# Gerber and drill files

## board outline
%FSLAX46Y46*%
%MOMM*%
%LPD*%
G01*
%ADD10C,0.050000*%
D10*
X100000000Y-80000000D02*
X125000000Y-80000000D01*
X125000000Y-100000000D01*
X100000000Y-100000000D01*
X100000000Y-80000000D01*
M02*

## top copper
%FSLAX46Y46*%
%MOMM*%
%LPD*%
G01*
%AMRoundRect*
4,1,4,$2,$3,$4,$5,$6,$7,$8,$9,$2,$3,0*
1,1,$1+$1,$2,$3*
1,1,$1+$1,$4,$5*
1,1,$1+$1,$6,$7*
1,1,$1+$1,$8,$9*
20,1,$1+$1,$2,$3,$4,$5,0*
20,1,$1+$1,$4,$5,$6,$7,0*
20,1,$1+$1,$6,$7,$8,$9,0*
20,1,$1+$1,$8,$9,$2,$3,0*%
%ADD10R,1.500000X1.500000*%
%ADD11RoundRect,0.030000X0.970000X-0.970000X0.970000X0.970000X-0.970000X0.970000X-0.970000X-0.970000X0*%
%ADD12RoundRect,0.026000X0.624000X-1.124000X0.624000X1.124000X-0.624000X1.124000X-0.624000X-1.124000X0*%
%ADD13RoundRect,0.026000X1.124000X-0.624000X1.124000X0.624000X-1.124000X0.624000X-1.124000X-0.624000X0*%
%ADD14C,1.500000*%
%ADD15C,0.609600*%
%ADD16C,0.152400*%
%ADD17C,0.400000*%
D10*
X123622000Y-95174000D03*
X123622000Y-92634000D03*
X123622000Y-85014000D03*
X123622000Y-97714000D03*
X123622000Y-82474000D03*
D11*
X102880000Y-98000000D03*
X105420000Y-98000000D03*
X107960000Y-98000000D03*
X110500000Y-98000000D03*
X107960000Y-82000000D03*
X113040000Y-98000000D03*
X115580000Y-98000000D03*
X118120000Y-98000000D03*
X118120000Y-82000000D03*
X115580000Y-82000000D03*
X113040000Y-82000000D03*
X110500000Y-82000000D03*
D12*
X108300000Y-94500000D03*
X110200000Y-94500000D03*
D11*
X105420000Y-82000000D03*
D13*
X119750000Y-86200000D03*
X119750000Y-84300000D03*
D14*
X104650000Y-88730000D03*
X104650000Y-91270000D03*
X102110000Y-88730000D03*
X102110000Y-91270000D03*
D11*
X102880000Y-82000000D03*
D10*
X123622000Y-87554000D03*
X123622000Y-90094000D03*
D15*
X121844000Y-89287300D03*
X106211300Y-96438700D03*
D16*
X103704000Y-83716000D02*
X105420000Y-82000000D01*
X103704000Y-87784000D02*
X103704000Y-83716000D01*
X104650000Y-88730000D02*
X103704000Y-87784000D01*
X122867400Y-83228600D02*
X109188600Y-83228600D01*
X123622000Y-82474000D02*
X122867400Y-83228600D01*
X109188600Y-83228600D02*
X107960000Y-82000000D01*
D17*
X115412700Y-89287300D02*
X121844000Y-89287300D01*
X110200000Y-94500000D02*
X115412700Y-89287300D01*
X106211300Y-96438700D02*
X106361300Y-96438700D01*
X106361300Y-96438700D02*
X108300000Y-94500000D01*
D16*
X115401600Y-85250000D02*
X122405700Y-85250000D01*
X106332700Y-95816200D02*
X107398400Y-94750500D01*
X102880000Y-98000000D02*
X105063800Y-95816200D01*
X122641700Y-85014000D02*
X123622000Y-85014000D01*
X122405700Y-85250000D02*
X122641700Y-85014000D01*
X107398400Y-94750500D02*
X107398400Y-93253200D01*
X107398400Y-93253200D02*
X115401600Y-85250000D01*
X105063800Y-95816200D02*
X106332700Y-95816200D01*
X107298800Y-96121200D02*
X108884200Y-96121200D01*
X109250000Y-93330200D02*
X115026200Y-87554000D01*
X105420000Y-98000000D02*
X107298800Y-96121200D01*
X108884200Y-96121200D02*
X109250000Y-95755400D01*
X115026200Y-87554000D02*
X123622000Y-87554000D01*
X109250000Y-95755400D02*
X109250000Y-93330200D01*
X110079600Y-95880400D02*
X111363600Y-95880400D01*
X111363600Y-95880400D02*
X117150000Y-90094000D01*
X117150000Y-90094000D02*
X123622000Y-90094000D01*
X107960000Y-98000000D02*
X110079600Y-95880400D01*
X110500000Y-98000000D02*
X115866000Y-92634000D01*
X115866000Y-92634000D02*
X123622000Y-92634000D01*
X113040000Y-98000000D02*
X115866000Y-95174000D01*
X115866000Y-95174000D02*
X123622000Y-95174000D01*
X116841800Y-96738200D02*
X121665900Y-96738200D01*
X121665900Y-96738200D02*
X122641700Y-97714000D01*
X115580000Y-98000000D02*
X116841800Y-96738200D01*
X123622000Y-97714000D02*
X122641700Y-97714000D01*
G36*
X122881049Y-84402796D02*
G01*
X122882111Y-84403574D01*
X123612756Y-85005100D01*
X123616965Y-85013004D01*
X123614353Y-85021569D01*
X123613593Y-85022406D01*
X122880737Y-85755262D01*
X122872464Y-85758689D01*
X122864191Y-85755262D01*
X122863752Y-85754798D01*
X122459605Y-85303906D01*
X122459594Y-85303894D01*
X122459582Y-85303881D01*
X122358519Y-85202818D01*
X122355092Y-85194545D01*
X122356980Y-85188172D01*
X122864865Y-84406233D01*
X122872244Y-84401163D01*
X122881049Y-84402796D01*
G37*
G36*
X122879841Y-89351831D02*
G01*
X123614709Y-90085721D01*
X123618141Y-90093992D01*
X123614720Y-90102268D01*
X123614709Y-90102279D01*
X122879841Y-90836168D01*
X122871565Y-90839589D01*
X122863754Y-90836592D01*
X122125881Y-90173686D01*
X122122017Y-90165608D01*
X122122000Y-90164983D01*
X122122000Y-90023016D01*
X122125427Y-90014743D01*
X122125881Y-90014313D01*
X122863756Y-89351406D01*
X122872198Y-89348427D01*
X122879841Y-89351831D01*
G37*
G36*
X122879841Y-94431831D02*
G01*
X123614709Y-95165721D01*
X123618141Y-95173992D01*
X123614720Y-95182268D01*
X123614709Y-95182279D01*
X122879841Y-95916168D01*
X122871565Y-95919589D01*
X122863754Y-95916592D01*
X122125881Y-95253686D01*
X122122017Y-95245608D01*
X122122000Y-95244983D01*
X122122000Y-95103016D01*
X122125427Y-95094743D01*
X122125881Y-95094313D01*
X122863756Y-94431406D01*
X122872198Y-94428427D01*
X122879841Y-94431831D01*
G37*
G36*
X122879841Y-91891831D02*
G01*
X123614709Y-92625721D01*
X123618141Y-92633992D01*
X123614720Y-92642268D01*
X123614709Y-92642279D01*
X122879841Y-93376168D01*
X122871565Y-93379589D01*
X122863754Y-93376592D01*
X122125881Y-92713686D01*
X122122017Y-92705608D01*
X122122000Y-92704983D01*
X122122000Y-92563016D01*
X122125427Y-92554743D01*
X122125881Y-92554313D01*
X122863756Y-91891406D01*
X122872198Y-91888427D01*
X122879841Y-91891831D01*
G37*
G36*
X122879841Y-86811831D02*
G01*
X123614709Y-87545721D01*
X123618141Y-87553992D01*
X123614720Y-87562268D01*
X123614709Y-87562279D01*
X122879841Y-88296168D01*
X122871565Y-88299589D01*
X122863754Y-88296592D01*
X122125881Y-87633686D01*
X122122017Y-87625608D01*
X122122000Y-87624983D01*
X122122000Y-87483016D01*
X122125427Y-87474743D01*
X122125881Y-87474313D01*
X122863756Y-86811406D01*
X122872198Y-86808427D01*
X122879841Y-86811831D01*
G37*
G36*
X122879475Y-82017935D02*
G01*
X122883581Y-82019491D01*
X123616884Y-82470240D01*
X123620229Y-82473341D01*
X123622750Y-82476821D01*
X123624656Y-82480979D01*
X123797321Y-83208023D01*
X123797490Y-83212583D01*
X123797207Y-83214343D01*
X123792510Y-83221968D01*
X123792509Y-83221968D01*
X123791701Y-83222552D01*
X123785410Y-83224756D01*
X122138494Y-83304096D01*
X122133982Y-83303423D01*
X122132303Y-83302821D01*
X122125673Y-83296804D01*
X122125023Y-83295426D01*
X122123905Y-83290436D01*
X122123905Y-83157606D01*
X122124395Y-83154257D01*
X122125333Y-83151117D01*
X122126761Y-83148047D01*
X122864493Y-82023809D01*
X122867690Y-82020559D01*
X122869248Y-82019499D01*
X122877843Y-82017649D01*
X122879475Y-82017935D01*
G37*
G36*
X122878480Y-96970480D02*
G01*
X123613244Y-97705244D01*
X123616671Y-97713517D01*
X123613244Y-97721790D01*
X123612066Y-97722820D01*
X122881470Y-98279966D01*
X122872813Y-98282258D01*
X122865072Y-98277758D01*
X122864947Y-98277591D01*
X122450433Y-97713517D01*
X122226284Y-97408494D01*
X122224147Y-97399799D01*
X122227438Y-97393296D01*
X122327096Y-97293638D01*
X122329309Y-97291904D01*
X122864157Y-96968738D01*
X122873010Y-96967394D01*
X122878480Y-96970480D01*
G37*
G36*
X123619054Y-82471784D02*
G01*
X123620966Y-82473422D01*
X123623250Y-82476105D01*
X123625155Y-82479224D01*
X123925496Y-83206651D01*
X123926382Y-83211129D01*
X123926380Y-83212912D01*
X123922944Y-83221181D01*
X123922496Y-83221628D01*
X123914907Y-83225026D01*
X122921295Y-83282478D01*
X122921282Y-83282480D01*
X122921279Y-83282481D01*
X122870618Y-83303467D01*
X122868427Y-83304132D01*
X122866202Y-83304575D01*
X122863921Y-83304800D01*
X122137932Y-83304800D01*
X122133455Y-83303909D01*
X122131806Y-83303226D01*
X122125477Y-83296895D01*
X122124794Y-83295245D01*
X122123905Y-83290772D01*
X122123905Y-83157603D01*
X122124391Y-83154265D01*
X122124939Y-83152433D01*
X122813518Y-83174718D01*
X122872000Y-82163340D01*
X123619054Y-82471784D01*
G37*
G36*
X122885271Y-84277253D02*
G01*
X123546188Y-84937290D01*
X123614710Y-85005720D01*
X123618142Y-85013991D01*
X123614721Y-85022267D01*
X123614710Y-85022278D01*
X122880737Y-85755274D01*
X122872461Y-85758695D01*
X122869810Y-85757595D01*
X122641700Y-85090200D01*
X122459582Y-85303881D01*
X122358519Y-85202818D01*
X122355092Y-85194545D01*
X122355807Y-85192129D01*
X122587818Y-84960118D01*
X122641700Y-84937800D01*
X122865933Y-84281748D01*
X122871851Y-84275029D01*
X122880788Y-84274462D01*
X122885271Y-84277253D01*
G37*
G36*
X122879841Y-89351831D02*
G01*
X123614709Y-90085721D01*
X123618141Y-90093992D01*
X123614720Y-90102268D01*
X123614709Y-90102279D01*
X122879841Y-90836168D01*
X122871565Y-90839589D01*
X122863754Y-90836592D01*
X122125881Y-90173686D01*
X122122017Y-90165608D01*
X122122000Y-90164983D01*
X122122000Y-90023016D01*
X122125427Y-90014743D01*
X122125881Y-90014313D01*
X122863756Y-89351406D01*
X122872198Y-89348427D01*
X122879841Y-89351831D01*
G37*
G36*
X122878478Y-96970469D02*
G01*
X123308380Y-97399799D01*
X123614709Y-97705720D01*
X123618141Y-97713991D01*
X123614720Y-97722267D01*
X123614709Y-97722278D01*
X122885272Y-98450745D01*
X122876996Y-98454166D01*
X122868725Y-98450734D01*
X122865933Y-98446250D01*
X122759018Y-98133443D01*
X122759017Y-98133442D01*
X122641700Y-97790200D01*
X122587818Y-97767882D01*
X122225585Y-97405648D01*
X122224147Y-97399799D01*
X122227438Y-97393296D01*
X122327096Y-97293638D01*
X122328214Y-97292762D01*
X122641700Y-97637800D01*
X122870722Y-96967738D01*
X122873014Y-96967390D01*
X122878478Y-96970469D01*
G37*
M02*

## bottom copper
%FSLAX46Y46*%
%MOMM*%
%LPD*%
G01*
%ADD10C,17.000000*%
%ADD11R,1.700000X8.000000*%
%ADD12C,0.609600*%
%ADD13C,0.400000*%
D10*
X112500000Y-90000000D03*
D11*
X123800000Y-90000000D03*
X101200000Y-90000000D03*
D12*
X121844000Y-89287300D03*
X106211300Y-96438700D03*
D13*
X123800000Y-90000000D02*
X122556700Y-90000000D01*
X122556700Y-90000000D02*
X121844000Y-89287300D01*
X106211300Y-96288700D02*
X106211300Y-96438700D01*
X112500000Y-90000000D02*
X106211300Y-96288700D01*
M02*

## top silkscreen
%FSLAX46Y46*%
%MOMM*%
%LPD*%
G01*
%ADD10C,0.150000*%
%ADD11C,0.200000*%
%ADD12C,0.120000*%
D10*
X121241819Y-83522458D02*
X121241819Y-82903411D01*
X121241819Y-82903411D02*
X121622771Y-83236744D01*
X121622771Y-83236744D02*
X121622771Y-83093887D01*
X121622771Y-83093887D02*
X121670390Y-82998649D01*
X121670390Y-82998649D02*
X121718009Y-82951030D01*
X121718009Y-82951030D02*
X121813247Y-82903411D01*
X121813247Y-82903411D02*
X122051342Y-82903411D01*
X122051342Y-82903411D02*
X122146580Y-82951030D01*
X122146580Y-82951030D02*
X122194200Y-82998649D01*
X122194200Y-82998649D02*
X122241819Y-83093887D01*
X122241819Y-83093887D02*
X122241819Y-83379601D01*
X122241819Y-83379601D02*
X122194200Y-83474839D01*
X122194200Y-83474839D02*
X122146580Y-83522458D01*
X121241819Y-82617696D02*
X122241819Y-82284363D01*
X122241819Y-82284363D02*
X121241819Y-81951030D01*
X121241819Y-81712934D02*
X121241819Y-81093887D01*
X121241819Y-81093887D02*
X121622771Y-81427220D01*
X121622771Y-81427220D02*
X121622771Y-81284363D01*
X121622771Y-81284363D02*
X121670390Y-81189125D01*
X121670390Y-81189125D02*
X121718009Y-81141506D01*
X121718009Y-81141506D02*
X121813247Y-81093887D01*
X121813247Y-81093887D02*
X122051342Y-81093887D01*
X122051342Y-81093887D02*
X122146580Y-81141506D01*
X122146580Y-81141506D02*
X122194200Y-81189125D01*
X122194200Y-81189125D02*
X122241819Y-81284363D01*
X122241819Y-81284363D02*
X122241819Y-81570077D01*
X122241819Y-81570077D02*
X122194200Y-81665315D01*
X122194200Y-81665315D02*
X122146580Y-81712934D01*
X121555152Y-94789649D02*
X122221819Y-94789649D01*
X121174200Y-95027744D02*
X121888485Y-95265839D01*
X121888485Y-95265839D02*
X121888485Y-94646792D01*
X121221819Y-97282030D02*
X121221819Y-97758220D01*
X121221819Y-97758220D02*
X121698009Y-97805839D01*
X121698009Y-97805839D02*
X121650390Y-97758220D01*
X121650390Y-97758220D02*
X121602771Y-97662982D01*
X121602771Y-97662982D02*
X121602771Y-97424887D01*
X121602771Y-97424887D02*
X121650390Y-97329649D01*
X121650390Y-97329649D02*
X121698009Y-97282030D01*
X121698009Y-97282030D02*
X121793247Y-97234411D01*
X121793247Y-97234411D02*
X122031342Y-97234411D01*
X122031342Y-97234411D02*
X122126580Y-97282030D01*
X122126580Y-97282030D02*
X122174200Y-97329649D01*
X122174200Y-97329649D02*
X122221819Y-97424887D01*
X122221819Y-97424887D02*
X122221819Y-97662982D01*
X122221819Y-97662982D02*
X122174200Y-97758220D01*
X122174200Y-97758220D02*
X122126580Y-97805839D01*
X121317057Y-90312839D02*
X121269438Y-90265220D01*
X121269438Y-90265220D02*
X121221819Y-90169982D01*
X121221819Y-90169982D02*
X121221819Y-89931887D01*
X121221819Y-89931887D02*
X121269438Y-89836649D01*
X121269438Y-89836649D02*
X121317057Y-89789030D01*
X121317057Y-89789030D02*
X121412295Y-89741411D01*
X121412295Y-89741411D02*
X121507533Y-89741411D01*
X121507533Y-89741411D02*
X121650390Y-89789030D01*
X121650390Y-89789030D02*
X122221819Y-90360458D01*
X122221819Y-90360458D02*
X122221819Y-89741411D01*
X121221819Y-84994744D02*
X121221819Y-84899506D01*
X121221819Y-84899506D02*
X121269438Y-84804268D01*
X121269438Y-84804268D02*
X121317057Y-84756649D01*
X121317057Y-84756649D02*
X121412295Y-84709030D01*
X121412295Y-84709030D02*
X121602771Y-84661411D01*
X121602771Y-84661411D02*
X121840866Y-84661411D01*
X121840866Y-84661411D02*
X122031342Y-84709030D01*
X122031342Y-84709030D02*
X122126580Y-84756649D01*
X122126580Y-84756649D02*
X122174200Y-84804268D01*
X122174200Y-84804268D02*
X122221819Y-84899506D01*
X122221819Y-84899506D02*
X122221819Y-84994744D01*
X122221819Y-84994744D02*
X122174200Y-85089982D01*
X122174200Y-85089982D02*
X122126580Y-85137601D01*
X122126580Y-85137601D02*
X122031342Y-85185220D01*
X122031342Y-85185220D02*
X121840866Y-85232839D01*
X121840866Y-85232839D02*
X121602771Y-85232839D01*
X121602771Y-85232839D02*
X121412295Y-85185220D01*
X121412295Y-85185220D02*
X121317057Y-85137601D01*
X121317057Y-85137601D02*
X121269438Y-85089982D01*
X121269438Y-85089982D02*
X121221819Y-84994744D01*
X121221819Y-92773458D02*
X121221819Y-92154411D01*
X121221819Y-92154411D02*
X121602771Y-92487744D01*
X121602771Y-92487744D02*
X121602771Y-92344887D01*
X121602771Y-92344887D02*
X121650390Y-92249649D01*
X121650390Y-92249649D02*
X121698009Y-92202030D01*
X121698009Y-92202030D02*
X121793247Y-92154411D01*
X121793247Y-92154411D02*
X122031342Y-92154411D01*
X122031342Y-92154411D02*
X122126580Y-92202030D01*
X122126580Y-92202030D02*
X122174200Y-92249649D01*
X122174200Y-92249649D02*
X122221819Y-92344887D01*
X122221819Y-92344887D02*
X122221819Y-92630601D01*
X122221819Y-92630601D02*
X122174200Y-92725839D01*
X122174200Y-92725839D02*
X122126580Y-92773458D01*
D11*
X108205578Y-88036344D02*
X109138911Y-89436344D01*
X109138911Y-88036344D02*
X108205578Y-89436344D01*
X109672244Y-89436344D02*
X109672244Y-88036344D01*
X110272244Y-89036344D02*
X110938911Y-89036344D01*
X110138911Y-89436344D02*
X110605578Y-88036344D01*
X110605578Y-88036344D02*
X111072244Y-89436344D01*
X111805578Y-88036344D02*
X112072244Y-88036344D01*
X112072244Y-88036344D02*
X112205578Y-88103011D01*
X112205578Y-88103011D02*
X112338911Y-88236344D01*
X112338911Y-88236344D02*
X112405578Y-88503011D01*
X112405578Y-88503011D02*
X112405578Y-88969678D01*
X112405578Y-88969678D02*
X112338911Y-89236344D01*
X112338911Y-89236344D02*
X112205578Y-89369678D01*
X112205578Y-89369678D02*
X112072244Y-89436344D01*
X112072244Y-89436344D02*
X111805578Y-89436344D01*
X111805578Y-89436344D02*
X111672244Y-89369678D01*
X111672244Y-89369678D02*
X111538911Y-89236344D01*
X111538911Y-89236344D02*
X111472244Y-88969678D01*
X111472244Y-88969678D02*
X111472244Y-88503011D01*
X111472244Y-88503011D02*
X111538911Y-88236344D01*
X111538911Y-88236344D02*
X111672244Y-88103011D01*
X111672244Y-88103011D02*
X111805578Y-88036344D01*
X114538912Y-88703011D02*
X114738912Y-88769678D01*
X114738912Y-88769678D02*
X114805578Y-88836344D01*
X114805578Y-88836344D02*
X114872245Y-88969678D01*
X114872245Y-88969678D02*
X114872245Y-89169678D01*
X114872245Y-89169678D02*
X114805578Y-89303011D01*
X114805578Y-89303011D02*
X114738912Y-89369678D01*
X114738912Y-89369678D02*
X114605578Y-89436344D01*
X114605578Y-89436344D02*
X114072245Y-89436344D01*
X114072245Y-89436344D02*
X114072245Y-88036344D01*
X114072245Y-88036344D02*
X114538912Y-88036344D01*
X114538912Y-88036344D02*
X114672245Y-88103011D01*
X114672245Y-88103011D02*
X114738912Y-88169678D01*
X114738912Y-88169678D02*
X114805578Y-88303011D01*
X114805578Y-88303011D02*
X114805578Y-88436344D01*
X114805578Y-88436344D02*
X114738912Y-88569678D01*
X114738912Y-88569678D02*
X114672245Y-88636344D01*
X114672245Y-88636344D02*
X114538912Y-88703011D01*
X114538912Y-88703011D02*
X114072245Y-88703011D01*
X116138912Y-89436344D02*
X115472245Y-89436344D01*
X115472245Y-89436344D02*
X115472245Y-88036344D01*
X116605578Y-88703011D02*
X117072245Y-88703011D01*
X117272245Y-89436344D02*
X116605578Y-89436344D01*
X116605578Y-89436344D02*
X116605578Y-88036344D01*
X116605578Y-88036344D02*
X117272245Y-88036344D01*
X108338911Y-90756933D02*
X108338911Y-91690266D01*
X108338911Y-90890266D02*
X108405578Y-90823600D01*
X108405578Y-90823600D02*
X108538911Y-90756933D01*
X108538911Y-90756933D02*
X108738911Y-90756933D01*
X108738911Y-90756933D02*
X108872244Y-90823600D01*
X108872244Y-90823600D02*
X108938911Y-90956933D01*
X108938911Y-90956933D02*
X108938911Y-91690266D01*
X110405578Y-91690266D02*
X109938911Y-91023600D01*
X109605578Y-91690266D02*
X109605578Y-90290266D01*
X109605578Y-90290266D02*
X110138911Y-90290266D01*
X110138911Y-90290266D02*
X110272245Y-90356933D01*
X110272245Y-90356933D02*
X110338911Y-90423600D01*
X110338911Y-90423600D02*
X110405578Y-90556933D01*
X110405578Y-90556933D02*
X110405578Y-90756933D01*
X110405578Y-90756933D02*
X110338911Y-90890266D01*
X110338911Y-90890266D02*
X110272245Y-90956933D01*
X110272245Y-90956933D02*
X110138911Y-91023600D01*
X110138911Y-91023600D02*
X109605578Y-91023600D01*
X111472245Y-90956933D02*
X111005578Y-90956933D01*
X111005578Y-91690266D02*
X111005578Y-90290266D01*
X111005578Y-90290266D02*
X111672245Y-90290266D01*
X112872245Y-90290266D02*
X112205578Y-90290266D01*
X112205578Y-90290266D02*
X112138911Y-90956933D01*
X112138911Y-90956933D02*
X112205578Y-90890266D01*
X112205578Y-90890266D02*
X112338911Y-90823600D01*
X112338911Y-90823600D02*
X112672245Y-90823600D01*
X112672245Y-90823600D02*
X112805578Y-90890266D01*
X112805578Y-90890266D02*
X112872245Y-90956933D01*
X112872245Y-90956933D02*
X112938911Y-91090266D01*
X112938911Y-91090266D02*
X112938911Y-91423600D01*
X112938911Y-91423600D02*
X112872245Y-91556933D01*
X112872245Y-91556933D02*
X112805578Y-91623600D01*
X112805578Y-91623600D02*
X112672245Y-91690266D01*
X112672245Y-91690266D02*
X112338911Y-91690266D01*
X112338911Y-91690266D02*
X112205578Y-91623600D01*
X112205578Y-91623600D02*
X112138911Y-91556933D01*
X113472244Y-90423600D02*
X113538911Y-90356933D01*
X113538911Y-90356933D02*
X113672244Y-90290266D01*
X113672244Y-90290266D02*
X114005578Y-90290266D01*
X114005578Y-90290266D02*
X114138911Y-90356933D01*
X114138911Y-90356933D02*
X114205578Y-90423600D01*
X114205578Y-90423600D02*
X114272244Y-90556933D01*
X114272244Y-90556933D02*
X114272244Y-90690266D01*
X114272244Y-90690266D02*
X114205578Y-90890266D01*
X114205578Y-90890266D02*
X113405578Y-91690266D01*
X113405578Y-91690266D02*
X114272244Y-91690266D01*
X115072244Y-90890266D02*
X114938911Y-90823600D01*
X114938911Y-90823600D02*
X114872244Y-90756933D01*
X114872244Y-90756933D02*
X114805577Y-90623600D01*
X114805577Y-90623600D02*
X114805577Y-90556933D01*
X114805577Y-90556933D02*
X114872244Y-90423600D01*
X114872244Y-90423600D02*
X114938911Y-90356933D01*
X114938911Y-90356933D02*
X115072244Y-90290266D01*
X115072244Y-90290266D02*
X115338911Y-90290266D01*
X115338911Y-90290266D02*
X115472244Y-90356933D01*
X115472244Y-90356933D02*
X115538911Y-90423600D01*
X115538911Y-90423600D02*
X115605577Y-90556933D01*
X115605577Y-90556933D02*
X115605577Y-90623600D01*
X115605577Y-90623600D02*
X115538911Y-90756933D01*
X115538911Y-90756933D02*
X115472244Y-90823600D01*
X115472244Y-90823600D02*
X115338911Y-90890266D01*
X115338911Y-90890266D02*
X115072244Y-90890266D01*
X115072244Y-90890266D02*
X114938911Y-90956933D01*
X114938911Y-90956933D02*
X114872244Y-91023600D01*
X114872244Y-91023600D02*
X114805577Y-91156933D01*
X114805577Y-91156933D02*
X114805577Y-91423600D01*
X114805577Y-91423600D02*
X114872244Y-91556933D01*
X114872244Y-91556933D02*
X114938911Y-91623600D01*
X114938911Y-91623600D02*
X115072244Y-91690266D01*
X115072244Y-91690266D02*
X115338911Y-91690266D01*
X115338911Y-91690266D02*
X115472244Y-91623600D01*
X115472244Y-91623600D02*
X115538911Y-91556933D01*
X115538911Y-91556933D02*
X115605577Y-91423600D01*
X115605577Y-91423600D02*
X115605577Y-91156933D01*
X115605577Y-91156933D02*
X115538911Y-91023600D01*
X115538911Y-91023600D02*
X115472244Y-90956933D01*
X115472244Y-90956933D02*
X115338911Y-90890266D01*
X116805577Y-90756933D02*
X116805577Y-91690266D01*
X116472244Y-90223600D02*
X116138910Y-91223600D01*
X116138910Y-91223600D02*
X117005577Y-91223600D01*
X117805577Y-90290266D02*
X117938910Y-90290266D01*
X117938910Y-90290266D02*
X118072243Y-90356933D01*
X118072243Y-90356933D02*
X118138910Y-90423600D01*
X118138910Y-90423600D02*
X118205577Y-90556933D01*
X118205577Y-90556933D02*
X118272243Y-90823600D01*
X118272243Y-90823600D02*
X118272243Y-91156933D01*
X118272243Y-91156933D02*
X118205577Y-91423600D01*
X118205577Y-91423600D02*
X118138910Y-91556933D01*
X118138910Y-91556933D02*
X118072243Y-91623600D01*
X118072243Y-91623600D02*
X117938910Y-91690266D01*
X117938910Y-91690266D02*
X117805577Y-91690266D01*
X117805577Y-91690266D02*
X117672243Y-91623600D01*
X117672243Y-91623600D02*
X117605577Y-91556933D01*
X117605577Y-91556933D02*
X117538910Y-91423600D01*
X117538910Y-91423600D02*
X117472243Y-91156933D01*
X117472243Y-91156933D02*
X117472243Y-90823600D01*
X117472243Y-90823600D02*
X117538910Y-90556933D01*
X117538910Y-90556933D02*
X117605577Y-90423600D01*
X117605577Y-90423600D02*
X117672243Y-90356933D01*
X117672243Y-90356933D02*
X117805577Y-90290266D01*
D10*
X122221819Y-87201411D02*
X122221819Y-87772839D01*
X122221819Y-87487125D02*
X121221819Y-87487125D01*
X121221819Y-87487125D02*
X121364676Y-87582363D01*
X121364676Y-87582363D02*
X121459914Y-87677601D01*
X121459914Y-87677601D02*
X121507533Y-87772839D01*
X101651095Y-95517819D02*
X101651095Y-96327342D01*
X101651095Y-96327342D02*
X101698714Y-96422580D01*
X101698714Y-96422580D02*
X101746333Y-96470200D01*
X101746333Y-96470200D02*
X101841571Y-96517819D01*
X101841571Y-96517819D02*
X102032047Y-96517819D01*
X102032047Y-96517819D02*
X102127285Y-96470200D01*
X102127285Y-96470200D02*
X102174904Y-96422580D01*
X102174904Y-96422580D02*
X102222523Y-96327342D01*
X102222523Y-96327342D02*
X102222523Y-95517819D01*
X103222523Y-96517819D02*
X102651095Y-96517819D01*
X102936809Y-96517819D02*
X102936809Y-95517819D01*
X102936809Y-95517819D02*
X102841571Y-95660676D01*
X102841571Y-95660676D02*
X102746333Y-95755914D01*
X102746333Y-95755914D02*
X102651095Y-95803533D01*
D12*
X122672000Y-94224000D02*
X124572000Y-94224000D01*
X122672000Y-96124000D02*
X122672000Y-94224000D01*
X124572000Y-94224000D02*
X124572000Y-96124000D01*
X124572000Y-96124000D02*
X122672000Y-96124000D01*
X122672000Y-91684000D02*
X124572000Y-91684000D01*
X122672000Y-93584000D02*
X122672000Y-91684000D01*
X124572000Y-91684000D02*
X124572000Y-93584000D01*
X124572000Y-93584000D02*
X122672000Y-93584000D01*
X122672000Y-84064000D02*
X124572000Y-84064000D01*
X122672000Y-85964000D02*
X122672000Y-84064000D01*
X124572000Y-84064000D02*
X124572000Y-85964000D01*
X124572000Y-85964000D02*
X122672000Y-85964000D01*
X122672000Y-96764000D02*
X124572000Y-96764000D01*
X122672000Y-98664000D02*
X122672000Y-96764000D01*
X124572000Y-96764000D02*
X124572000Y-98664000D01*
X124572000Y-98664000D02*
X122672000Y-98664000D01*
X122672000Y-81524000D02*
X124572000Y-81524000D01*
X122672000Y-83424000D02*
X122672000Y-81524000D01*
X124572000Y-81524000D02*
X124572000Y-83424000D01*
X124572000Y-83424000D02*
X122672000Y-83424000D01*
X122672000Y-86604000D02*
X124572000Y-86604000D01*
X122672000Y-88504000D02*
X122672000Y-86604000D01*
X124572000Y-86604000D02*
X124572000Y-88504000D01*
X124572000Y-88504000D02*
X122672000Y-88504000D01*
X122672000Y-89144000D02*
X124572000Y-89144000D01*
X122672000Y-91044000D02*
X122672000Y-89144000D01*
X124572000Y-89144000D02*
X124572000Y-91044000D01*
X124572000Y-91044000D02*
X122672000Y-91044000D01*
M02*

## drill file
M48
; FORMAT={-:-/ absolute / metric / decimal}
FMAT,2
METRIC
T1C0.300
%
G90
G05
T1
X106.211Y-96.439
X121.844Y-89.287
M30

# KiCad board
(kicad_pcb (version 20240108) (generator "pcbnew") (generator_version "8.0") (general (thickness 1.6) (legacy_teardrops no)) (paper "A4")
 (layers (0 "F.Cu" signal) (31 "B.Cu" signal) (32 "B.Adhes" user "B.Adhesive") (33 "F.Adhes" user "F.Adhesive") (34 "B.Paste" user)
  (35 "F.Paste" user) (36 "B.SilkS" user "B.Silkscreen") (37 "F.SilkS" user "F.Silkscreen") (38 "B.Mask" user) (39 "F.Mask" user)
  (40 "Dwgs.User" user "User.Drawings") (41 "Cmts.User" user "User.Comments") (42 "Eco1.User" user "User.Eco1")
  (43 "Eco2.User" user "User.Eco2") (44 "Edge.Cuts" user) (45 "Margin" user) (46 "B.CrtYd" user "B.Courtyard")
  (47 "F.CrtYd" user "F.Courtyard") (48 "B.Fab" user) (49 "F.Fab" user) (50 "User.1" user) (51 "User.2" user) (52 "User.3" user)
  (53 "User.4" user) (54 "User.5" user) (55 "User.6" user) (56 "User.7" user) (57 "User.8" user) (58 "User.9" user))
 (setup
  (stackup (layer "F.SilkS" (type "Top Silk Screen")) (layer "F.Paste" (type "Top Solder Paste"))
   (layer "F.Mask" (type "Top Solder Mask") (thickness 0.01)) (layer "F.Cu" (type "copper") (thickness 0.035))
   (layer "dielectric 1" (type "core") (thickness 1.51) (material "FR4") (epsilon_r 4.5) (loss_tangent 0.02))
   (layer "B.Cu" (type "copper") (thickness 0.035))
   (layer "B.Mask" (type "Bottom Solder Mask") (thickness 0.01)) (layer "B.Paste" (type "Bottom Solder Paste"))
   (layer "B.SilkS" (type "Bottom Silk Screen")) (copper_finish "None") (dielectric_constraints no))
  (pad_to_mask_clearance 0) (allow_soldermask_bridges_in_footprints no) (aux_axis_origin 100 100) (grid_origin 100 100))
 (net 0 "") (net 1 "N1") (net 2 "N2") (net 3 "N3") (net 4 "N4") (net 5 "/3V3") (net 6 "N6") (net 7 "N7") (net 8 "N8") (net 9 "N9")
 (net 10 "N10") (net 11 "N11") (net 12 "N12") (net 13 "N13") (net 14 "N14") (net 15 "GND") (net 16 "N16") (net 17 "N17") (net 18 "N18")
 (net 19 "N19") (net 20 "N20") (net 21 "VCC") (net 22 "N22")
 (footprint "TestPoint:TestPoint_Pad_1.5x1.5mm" (layer "F.Cu") (at 123.622 95.174)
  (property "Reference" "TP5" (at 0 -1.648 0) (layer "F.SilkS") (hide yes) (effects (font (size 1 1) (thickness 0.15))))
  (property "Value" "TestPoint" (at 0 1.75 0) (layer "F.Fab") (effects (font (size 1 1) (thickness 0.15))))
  (fp_line (start -0.95 -0.95) (end 0.95 -0.95) (stroke (width 0.12) (type solid)) (layer "F.SilkS"))
  (fp_line (start -0.95 0.95) (end -0.95 -0.95) (stroke (width 0.12) (type solid)) (layer "F.SilkS"))
  (fp_line (start 0.95 -0.95) (end 0.95 0.95) (stroke (width 0.12) (type solid)) (layer "F.SilkS"))
  (fp_line (start 0.95 0.95) (end -0.95 0.95) (stroke (width 0.12) (type solid)) (layer "F.SilkS"))
  (pad "1" smd rect (at 0 0) (size 1.5 1.5) (layers "F.Cu" "F.Mask") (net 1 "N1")
   (teardrops (best_length_ratio 0.5) (max_length 1) (best_width_ratio 1) (max_width 2) (curve_points 0) (filter_ratio 0.9) (enabled yes)
    (allow_two_segments yes) (prefer_zone_connections yes))))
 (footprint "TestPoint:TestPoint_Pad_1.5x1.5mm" (layer "F.Cu") (at 123.622 92.634)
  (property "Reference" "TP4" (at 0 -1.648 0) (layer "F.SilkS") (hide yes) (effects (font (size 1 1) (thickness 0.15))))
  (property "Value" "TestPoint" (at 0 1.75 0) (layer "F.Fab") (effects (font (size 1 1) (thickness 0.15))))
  (fp_line (start -0.95 -0.95) (end 0.95 -0.95) (stroke (width 0.12) (type solid)) (layer "F.SilkS"))
  (fp_line (start -0.95 0.95) (end -0.95 -0.95) (stroke (width 0.12) (type solid)) (layer "F.SilkS"))
  (fp_line (start 0.95 -0.95) (end 0.95 0.95) (stroke (width 0.12) (type solid)) (layer "F.SilkS"))
  (fp_line (start 0.95 0.95) (end -0.95 0.95) (stroke (width 0.12) (type solid)) (layer "F.SilkS"))
  (pad "1" smd rect (at 0 0) (size 1.5 1.5) (layers "F.Cu" "F.Mask") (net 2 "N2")
   (teardrops (best_length_ratio 0.5) (max_length 1) (best_width_ratio 1) (max_width 2) (curve_points 0) (filter_ratio 0.9) (enabled yes)
    (allow_two_segments yes) (prefer_zone_connections yes))))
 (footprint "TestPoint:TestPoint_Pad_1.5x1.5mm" (layer "F.Cu") (at 123.622 85.014)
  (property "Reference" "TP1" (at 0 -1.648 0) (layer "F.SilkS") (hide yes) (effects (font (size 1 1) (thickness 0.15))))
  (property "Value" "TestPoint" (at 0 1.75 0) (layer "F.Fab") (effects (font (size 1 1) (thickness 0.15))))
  (fp_line (start -0.95 -0.95) (end 0.95 -0.95) (stroke (width 0.12) (type solid)) (layer "F.SilkS"))
  (fp_line (start -0.95 0.95) (end -0.95 -0.95) (stroke (width 0.12) (type solid)) (layer "F.SilkS"))
  (fp_line (start 0.95 -0.95) (end 0.95 0.95) (stroke (width 0.12) (type solid)) (layer "F.SilkS"))
  (fp_line (start 0.95 0.95) (end -0.95 0.95) (stroke (width 0.12) (type solid)) (layer "F.SilkS"))
  (pad "1" smd rect (at 0 0) (size 1.5 1.5) (layers "F.Cu" "F.Mask") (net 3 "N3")
   (teardrops (best_length_ratio 0.5) (max_length 1) (best_width_ratio 1) (max_width 2) (curve_points 0) (filter_ratio 0.9) (enabled yes)
    (allow_two_segments yes) (prefer_zone_connections yes))))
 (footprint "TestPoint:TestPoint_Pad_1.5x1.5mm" (layer "F.Cu") (at 123.622 97.714)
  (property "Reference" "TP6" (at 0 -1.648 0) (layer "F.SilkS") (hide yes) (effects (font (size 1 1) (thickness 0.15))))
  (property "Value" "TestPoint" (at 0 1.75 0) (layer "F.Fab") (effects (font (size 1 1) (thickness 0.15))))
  (fp_line (start -0.95 -0.95) (end 0.95 -0.95) (stroke (width 0.12) (type solid)) (layer "F.SilkS"))
  (fp_line (start -0.95 0.95) (end -0.95 -0.95) (stroke (width 0.12) (type solid)) (layer "F.SilkS"))
  (fp_line (start 0.95 -0.95) (end 0.95 0.95) (stroke (width 0.12) (type solid)) (layer "F.SilkS"))
  (fp_line (start 0.95 0.95) (end -0.95 0.95) (stroke (width 0.12) (type solid)) (layer "F.SilkS"))
  (pad "1" smd rect (at 0 0) (size 1.5 1.5) (layers "F.Cu" "F.Mask") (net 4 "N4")
   (teardrops (best_length_ratio 0.5) (max_length 1) (best_width_ratio 1) (max_width 2) (curve_points 0) (filter_ratio 0.9) (enabled yes)
    (allow_two_segments yes) (prefer_zone_connections yes))))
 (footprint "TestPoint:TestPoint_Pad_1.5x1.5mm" (layer "F.Cu") (at 123.622 82.474)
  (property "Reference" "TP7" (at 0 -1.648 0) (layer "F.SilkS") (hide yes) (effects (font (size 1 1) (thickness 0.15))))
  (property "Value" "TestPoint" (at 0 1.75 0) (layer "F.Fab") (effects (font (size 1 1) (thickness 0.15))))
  (fp_line (start -0.95 -0.95) (end 0.95 -0.95) (stroke (width 0.12) (type solid)) (layer "F.SilkS"))
  (fp_line (start -0.95 0.95) (end -0.95 -0.95) (stroke (width 0.12) (type solid)) (layer "F.SilkS"))
  (fp_line (start 0.95 -0.95) (end 0.95 0.95) (stroke (width 0.12) (type solid)) (layer "F.SilkS"))
  (fp_line (start 0.95 0.95) (end -0.95 0.95) (stroke (width 0.12) (type solid)) (layer "F.SilkS"))
  (pad "1" smd rect (at 0 0) (size 1.5 1.5) (layers "F.Cu" "F.Mask") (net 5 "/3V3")
   (teardrops (best_length_ratio 0.5) (max_length 1) (best_width_ratio 1) (max_width 2) (curve_points 0) (filter_ratio 0.9) (enabled yes)
    (allow_two_segments yes) (prefer_zone_connections yes))))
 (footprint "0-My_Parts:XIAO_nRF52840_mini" (layer "F.Cu") (at 110.5 90 90)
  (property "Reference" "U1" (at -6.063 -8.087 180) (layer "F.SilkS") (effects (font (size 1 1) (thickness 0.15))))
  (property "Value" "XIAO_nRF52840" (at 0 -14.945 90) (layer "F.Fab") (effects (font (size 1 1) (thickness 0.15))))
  (pad "0" smd roundrect (at -8 -7.62 90) (size 2 2) (layers "F.Cu" "F.Paste" "F.Mask") (roundrect_rratio 0.015) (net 3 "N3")
   (solder_mask_margin 0.102))
  (pad "1" smd roundrect (at -8 -5.08 90) (size 2 2) (layers "F.Cu" "F.Paste" "F.Mask") (roundrect_rratio 0.015) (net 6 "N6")
   (solder_mask_margin 0.102))
  (pad "2" smd roundrect (at -8 -2.54 90) (size 2 2) (layers "F.Cu" "F.Paste" "F.Mask") (roundrect_rratio 0.015) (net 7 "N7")
   (solder_mask_margin 0.102))
  (pad "3" smd roundrect (at -8 0 90) (size 2 2) (layers "F.Cu" "F.Paste" "F.Mask") (roundrect_rratio 0.015) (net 2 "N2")
   (solder_mask_margin 0.102))
  (pad "3V3" smd roundrect (at 8 -2.54 90) (size 2 2) (layers "F.Cu" "F.Paste" "F.Mask") (roundrect_rratio 0.015) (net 5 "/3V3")
   (solder_mask_margin 0.102))
  (pad "4" smd roundrect (at -8 2.54 90) (size 2 2) (layers "F.Cu" "F.Paste" "F.Mask") (roundrect_rratio 0.015) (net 1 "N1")
   (solder_mask_margin 0.102))
  (pad "5" smd roundrect (at -8 5.08 90) (size 2 2) (layers "F.Cu" "F.Paste" "F.Mask") (roundrect_rratio 0.015) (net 4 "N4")
   (solder_mask_margin 0.102))
  (pad "6" smd roundrect (at -8 7.62 90) (size 2 2) (layers "F.Cu" "F.Paste" "F.Mask") (roundrect_rratio 0.015) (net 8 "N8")
   (solder_mask_margin 0.102))
  (pad "7" smd roundrect (at 8 7.62 90) (size 2 2) (layers "F.Cu" "F.Paste" "F.Mask") (roundrect_rratio 0.015) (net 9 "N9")
   (solder_mask_margin 0.102))
  (pad "8" smd roundrect (at 8 5.08 90) (size 2 2) (layers "F.Cu" "F.Paste" "F.Mask") (roundrect_rratio 0.015) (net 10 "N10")
   (solder_mask_margin 0.102))
  (pad "9" smd roundrect (at 8 2.54 90) (size 2 2) (layers "F.Cu" "F.Paste" "F.Mask") (roundrect_rratio 0.015) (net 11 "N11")
   (solder_mask_margin 0.102))
  (pad "10" smd roundrect (at 8 0 90) (size 2 2) (layers "F.Cu" "F.Paste" "F.Mask") (roundrect_rratio 0.015) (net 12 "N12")
   (solder_mask_margin 0.102))
  (pad "BAT_N" smd roundrect (at -4.5 -2.2 90) (size 2.3 1.3) (layers "F.Cu" "F.Paste" "F.Mask") (roundrect_rratio 0.02) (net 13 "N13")
   (solder_mask_margin 0.102))
  (pad "BAT_P" smd roundrect (at -4.5 -0.3 90) (size 2.3 1.3) (layers "F.Cu" "F.Paste" "F.Mask") (roundrect_rratio 0.02) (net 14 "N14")
   (solder_mask_margin 0.102))
  (pad "GND" smd roundrect (at 8 -5.08 90) (size 2 2) (layers "F.Cu" "F.Paste" "F.Mask") (roundrect_rratio 0.015) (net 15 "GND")
   (solder_mask_margin 0.102))
  (pad "NFC1" smd roundrect (at 3.8 9.25 90) (size 1.3 2.3) (layers "F.Cu" "F.Paste" "F.Mask") (roundrect_rratio 0.02) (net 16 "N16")
   (solder_mask_margin 0.102))
  (pad "NFC2" smd roundrect (at 5.7 9.25 90) (size 1.3 2.3) (layers "F.Cu" "F.Paste" "F.Mask") (roundrect_rratio 0.02) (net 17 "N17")
   (solder_mask_margin 0.102))
  (pad "TP1" smd circle (at 1.27 -5.85 90) (size 1.5 1.5) (layers "F.Cu" "F.Paste" "F.Mask") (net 15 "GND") (solder_mask_margin 0.102))
  (pad "TP2" smd circle (at -1.27 -5.85 90) (size 1.5 1.5) (layers "F.Cu" "F.Paste" "F.Mask") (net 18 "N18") (solder_mask_margin 0.102))
  (pad "TP3" smd circle (at 1.27 -8.39 90) (size 1.5 1.5) (layers "F.Cu" "F.Paste" "F.Mask") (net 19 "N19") (solder_mask_margin 0.102))
  (pad "TP5" smd circle (at -1.27 -8.39 90) (size 1.5 1.5) (layers "F.Cu" "F.Paste" "F.Mask") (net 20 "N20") (solder_mask_margin 0.102))
  (pad "VUSB" smd roundrect (at 8 -7.62 90) (size 2 2) (layers "F.Cu" "F.Paste" "F.Mask") (roundrect_rratio 0.015) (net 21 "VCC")
   (solder_mask_margin 0.102))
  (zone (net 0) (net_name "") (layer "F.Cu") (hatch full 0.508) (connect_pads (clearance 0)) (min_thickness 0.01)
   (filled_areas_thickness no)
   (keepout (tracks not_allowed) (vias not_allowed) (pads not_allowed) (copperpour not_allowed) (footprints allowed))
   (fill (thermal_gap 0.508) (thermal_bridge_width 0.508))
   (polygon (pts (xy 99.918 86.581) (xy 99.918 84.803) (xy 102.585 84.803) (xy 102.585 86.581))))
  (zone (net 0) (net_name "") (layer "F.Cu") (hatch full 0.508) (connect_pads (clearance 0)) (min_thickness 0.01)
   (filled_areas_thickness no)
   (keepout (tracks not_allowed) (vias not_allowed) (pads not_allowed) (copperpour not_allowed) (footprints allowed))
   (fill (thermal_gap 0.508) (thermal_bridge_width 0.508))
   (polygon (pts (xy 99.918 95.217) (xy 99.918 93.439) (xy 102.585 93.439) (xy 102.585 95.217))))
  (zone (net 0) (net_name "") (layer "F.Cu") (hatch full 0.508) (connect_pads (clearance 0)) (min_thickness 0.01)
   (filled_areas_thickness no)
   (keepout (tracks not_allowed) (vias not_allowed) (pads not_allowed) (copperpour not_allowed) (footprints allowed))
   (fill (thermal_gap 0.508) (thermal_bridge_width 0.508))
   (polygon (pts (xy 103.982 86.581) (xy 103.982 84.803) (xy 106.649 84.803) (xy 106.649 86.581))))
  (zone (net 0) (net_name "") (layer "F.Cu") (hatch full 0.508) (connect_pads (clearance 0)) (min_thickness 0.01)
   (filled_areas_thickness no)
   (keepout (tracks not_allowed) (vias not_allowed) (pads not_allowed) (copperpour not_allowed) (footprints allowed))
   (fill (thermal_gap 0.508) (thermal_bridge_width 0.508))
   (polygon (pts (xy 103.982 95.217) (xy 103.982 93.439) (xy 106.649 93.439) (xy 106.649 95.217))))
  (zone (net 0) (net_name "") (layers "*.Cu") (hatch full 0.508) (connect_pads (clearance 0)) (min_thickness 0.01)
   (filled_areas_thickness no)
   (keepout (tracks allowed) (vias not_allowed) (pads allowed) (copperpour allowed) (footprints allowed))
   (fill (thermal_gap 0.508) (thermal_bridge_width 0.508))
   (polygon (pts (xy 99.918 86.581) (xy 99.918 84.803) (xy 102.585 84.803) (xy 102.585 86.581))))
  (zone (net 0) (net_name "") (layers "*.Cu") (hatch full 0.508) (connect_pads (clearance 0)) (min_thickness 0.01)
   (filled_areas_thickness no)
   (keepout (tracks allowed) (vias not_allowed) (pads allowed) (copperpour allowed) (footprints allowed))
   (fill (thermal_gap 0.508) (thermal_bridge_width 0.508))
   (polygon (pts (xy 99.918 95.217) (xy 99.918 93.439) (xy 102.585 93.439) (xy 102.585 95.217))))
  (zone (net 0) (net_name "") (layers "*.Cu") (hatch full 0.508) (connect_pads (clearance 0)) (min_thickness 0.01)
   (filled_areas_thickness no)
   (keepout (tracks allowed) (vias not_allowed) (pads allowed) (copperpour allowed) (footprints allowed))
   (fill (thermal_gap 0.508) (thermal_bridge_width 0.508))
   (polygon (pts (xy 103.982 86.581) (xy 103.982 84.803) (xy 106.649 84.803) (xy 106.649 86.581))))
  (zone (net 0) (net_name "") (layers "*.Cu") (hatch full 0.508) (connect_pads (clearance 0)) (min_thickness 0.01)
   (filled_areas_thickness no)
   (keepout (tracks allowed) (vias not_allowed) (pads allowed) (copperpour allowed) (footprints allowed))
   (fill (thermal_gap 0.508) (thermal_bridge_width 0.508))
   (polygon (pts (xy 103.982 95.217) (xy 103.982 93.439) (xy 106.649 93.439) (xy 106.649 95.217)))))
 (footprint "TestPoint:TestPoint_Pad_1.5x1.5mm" (layer "F.Cu") (at 123.622 87.554)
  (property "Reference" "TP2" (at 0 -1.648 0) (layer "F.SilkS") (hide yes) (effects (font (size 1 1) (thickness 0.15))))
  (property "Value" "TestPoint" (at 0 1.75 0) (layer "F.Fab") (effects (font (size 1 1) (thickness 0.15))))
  (fp_line (start -0.95 -0.95) (end 0.95 -0.95) (stroke (width 0.12) (type solid)) (layer "F.SilkS"))
  (fp_line (start -0.95 0.95) (end -0.95 -0.95) (stroke (width 0.12) (type solid)) (layer "F.SilkS"))
  (fp_line (start 0.95 -0.95) (end 0.95 0.95) (stroke (width 0.12) (type solid)) (layer "F.SilkS"))
  (fp_line (start 0.95 0.95) (end -0.95 0.95) (stroke (width 0.12) (type solid)) (layer "F.SilkS"))
  (pad "1" smd rect (at 0 0) (size 1.5 1.5) (layers "F.Cu" "F.Mask") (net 6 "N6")
   (teardrops (best_length_ratio 0.5) (max_length 1) (best_width_ratio 1) (max_width 2) (curve_points 0) (filter_ratio 0.9) (enabled yes)
    (allow_two_segments yes) (prefer_zone_connections yes))))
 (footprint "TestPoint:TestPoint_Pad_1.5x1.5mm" (layer "F.Cu") (at 123.622 90.094)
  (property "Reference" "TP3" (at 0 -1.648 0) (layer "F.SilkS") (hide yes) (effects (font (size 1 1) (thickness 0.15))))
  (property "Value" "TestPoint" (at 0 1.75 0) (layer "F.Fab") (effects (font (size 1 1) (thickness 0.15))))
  (fp_line (start -0.95 -0.95) (end 0.95 -0.95) (stroke (width 0.12) (type solid)) (layer "F.SilkS"))
  (fp_line (start -0.95 0.95) (end -0.95 -0.95) (stroke (width 0.12) (type solid)) (layer "F.SilkS"))
  (fp_line (start 0.95 -0.95) (end 0.95 0.95) (stroke (width 0.12) (type solid)) (layer "F.SilkS"))
  (fp_line (start 0.95 0.95) (end -0.95 0.95) (stroke (width 0.12) (type solid)) (layer "F.SilkS"))
  (pad "1" smd rect (at 0 0) (size 1.5 1.5) (layers "F.Cu" "F.Mask") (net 7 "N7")
   (teardrops (best_length_ratio 0.5) (max_length 1) (best_width_ratio 1) (max_width 2) (curve_points 0) (filter_ratio 0.9) (enabled yes)
    (allow_two_segments yes) (prefer_zone_connections yes))))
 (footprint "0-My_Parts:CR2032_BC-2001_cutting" (layer "B.Cu") (at 112.5 90 180)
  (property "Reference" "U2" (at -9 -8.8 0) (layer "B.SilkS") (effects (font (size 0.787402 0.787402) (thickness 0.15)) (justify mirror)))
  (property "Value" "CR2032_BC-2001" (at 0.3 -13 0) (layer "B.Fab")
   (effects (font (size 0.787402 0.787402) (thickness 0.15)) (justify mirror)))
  (pad "P$1" smd circle (at 0 0 180) (size 17 17) (layers "B.Cu" "B.Paste" "B.Mask") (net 13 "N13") (solder_mask_margin 0.102))
  (pad "P$2" smd rect (at -11.3 0 180) (size 1.7 8) (layers "B.Cu" "B.Paste" "B.Mask") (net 14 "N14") (solder_mask_margin 0.102))
  (pad "P$3" smd rect (at 11.3 0 180) (size 1.7 8) (layers "B.Cu" "B.Paste" "B.Mask") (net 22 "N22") (solder_mask_margin 0.102)))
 (gr_rect (start 100 80) (end 125 100) (stroke (width 0.05) (type default)) (fill none) (layer "Edge.Cuts"))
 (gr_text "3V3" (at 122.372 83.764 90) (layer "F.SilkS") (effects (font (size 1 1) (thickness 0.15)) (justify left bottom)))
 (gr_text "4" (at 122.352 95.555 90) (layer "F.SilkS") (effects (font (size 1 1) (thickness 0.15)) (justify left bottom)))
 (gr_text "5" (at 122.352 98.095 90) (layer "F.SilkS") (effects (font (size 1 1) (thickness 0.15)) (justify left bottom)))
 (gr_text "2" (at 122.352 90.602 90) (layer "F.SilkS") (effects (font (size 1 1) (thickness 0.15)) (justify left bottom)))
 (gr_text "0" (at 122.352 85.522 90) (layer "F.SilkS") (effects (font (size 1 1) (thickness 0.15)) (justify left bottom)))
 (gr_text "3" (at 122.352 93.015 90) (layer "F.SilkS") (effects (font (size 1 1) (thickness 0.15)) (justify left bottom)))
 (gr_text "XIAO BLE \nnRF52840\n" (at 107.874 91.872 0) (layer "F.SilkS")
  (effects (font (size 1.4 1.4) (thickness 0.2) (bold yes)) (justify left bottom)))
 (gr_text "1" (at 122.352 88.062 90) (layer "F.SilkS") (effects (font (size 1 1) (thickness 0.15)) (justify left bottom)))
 (segment (start 103.704 83.716) (end 105.42 82) (width 0.1524) (layer "F.Cu") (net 15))
 (segment (start 103.704 87.784) (end 103.704 83.716) (width 0.1524) (layer "F.Cu") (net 15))
 (segment (start 104.65 88.73) (end 103.704 87.784) (width 0.1524) (layer "F.Cu") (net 15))
 (segment (start 122.8674 83.2286) (end 109.1886 83.2286) (width 0.1524) (layer "F.Cu") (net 5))
 (segment (start 123.622 82.474) (end 122.8674 83.2286) (width 0.1524) (layer "F.Cu") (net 5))
 (segment (start 109.1886 83.2286) (end 107.96 82) (width 0.1524) (layer "F.Cu") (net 5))
 (segment (start 115.4127 89.2873) (end 121.844 89.2873) (width 0.4) (layer "F.Cu") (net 14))
 (segment (start 110.2 94.5) (end 115.4127 89.2873) (width 0.4) (layer "F.Cu") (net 14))
 (via (at 121.844 89.2873) (size 0.6096) (drill 0.3) (layers "F.Cu" "B.Cu") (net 14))
 (segment (start 123.8 90) (end 122.5567 90) (width 0.4) (layer "B.Cu") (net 14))
 (segment (start 122.5567 90) (end 121.844 89.2873) (width 0.4) (layer "B.Cu") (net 14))
 (segment (start 106.2113 96.4387) (end 106.3613 96.4387) (width 0.4) (layer "F.Cu") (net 13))
 (segment (start 106.3613 96.4387) (end 108.3 94.5) (width 0.4) (layer "F.Cu") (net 13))
 (via (at 106.2113 96.4387) (size 0.6096) (drill 0.3) (layers "F.Cu" "B.Cu") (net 13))
 (segment (start 106.2113 96.2887) (end 106.2113 96.4387) (width 0.4) (layer "B.Cu") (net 13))
 (segment (start 112.5 90) (end 106.2113 96.2887) (width 0.4) (layer "B.Cu") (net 13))
 (segment (start 115.4016 85.25) (end 122.4057 85.25) (width 0.1524) (layer "F.Cu") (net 3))
 (segment (start 106.3327 95.8162) (end 107.3984 94.7505) (width 0.1524) (layer "F.Cu") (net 3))
 (segment (start 102.88 98) (end 105.0638 95.8162) (width 0.1524) (layer "F.Cu") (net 3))
 (segment (start 122.6417 85.014) (end 123.622 85.014) (width 0.1524) (layer "F.Cu") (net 3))
 (segment (start 122.4057 85.25) (end 122.6417 85.014) (width 0.1524) (layer "F.Cu") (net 3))
 (segment (start 107.3984 94.7505) (end 107.3984 93.2532) (width 0.1524) (layer "F.Cu") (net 3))
 (segment (start 107.3984 93.2532) (end 115.4016 85.25) (width 0.1524) (layer "F.Cu") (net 3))
 (segment (start 105.0638 95.8162) (end 106.3327 95.8162) (width 0.1524) (layer "F.Cu") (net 3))
 (segment (start 107.2988 96.1212) (end 108.8842 96.1212) (width 0.1524) (layer "F.Cu") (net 6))
 (segment (start 109.25 93.3302) (end 115.0262 87.554) (width 0.1524) (layer "F.Cu") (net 6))
 (segment (start 105.42 98) (end 107.2988 96.1212) (width 0.1524) (layer "F.Cu") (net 6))
 (segment (start 108.8842 96.1212) (end 109.25 95.7554) (width 0.1524) (layer "F.Cu") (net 6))
 (segment (start 115.0262 87.554) (end 123.622 87.554) (width 0.1524) (layer "F.Cu") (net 6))
 (segment (start 109.25 95.7554) (end 109.25 93.3302) (width 0.1524) (layer "F.Cu") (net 6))
 (segment (start 110.0796 95.8804) (end 111.3636 95.8804) (width 0.1524) (layer "F.Cu") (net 7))
 (segment (start 111.3636 95.8804) (end 117.15 90.094) (width 0.1524) (layer "F.Cu") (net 7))
 (segment (start 117.15 90.094) (end 123.622 90.094) (width 0.1524) (layer "F.Cu") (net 7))
 (segment (start 107.96 98) (end 110.0796 95.8804) (width 0.1524) (layer "F.Cu") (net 7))
 (segment (start 110.5 98) (end 115.866 92.634) (width 0.1524) (layer "F.Cu") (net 2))
 (segment (start 115.866 92.634) (end 123.622 92.634) (width 0.1524) (layer "F.Cu") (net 2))
 (segment (start 113.04 98) (end 115.866 95.174) (width 0.1524) (layer "F.Cu") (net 1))
 (segment (start 115.866 95.174) (end 123.622 95.174) (width 0.1524) (layer "F.Cu") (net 1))
 (segment (start 116.8418 96.7382) (end 121.6659 96.7382) (width 0.1524) (layer "F.Cu") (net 4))
 (segment (start 121.6659 96.7382) (end 122.6417 97.714) (width 0.1524) (layer "F.Cu") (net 4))
 (segment (start 115.58 98) (end 116.8418 96.7382) (width 0.1524) (layer "F.Cu") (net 4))
 (segment (start 123.622 97.714) (end 122.6417 97.714) (width 0.1524) (layer "F.Cu") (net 4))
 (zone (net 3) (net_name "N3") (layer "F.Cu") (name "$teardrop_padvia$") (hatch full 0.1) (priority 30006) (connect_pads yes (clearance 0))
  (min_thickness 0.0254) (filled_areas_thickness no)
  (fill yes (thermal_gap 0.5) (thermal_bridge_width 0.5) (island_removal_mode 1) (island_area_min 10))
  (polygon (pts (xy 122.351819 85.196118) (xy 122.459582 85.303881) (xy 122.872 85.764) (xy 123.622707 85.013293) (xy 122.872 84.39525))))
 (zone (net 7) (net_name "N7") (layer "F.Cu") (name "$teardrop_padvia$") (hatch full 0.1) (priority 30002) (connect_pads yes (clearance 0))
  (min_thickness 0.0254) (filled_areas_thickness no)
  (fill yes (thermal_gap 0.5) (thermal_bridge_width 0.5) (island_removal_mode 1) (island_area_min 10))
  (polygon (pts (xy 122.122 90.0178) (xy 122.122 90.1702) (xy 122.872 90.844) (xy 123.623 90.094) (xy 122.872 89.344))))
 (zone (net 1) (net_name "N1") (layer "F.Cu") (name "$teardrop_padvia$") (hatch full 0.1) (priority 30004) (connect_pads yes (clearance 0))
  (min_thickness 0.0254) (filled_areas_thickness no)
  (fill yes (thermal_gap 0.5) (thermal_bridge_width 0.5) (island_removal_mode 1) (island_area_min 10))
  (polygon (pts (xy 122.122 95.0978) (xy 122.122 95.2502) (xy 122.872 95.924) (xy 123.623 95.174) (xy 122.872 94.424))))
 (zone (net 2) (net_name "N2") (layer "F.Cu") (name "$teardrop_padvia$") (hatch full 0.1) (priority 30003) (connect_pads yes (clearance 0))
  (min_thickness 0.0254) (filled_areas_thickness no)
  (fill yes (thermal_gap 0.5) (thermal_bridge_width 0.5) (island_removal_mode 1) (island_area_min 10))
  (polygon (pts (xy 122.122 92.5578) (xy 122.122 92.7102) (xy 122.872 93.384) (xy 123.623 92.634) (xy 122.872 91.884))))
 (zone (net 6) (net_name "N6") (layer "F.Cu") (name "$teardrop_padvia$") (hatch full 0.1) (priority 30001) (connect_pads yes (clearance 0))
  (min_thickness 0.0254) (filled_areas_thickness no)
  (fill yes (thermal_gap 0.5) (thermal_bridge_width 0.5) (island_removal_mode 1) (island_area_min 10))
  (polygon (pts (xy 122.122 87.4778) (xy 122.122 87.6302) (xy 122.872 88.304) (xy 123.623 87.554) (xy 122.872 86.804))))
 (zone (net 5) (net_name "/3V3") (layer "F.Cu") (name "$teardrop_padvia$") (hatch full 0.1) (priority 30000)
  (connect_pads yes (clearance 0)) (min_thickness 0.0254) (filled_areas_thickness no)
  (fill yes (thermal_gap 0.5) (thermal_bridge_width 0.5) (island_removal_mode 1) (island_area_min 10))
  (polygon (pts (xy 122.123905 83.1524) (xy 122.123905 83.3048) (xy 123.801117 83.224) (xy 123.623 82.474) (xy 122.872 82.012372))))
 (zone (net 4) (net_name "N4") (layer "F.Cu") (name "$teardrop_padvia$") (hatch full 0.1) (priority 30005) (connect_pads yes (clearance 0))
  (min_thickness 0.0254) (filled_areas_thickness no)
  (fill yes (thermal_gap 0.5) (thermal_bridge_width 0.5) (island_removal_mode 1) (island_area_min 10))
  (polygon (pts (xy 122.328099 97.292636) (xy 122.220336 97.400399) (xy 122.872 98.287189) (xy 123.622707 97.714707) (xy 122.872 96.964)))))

